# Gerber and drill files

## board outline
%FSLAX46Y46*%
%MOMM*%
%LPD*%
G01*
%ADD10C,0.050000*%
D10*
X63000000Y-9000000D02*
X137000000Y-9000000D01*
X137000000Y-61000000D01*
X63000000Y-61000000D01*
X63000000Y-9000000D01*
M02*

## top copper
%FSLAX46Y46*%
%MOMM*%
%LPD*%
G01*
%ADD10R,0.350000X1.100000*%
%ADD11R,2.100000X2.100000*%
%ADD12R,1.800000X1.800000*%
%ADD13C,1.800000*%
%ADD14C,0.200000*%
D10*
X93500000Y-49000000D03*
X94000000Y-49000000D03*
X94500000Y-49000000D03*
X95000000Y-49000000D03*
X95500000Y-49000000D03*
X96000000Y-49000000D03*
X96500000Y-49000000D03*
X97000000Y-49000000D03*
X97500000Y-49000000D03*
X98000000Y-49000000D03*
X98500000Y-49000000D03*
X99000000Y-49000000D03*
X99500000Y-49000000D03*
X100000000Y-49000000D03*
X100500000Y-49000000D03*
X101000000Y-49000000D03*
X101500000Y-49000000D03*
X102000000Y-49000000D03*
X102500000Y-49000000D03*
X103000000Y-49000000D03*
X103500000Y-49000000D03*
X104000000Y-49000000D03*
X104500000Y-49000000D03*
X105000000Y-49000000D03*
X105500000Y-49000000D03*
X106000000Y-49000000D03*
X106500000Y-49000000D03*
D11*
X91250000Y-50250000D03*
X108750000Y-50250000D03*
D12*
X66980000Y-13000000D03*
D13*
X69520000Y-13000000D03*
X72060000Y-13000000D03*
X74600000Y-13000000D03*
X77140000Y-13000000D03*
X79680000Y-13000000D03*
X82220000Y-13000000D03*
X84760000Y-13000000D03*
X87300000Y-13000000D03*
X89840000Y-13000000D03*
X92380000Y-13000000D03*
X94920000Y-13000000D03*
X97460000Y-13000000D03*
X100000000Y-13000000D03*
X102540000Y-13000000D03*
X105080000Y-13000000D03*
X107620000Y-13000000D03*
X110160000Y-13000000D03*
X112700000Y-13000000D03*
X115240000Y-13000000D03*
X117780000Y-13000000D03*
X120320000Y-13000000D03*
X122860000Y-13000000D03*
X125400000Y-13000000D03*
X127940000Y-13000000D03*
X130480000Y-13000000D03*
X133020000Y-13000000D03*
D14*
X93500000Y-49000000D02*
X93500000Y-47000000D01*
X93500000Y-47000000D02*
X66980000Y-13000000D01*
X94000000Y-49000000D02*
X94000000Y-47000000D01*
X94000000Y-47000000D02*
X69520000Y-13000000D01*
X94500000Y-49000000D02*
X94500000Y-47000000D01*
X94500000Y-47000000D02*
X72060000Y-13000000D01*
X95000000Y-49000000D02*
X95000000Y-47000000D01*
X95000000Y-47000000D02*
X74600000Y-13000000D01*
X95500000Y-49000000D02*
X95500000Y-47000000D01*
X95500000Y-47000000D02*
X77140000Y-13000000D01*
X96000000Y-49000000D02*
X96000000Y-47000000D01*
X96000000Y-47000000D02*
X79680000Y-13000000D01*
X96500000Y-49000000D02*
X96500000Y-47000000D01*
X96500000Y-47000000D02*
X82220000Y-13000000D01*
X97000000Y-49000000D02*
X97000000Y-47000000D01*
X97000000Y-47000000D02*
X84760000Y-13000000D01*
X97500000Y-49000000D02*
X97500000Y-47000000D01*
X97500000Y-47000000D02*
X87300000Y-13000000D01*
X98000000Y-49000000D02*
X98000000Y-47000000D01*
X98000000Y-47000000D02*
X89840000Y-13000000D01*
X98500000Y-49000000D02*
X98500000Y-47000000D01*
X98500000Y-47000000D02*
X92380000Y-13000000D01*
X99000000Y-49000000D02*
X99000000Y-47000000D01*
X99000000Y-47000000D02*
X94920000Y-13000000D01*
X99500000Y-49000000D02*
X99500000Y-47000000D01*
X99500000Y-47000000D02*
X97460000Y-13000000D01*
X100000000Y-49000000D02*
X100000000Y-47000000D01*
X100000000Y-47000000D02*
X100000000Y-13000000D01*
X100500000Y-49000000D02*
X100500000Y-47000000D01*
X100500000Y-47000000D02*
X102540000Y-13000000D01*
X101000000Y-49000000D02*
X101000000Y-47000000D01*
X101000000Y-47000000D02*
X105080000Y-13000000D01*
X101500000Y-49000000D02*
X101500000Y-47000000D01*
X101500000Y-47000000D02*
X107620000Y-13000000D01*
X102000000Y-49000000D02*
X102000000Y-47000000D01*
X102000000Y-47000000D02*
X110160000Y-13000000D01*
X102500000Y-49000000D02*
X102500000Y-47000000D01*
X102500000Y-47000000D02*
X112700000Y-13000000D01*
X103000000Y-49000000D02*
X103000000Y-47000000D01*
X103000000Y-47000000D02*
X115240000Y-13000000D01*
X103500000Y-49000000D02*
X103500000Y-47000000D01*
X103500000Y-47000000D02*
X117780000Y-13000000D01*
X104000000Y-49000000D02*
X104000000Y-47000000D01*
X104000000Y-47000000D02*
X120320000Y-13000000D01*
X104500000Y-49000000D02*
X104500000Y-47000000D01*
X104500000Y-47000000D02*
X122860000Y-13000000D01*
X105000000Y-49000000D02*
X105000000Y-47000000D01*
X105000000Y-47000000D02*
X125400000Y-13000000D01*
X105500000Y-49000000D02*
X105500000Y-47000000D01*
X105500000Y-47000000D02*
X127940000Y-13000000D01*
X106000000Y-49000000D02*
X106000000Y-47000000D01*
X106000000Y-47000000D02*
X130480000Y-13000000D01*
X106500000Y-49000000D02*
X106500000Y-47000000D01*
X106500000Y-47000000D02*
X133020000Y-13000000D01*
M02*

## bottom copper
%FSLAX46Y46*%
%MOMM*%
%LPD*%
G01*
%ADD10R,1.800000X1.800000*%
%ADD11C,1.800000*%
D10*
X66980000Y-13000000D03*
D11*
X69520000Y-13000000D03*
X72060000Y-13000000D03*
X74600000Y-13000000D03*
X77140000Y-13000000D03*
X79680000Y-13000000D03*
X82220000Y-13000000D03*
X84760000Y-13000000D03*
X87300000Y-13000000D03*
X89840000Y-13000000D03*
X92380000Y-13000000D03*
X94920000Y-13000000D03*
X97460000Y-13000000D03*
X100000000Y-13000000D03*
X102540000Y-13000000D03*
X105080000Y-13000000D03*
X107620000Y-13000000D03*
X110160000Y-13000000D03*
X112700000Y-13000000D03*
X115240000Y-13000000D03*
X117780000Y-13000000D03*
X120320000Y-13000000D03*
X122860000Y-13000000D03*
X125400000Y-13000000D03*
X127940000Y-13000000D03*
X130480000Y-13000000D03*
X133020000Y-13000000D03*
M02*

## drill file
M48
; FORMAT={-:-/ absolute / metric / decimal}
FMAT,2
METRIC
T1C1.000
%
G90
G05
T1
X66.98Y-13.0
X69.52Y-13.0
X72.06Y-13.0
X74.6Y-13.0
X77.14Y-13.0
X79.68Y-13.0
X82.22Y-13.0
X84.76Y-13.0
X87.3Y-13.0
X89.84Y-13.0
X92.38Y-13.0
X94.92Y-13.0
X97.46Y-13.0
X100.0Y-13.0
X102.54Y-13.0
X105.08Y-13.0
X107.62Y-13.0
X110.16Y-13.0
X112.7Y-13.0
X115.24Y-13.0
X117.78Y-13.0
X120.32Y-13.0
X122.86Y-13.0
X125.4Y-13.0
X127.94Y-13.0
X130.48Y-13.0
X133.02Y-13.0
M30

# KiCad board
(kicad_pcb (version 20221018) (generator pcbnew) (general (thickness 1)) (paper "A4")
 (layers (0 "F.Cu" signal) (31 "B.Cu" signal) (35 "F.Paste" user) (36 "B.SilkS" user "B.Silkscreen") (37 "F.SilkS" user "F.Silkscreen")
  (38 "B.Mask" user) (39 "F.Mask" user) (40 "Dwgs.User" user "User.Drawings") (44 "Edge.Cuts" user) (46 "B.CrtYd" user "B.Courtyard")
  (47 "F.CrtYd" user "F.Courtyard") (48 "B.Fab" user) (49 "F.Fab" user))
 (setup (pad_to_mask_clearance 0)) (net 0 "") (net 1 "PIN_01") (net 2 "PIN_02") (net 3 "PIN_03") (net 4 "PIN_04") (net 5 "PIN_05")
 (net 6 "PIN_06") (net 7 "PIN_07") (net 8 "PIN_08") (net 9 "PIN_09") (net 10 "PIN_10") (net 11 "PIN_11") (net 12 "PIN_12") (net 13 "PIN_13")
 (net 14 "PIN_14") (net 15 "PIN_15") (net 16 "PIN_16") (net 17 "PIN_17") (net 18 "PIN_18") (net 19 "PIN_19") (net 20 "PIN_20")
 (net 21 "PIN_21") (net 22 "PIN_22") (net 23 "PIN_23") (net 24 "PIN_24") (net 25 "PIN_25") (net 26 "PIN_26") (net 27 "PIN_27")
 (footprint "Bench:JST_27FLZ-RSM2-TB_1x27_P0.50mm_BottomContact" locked (layer "F.Cu") (at 100 49)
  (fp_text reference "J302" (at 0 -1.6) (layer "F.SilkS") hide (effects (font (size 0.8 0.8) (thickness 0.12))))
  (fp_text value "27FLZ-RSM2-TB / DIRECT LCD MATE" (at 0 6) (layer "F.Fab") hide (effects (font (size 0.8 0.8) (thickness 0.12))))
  (pad "1" smd rect locked (at -6.5 0) (size 0.35 1.1) (layers "F.Cu" "F.Paste" "F.Mask") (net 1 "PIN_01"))
  (pad "2" smd rect locked (at -6 0) (size 0.35 1.1) (layers "F.Cu" "F.Paste" "F.Mask") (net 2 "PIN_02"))
  (pad "3" smd rect locked (at -5.5 0) (size 0.35 1.1) (layers "F.Cu" "F.Paste" "F.Mask") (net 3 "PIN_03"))
  (pad "4" smd rect locked (at -5 0) (size 0.35 1.1) (layers "F.Cu" "F.Paste" "F.Mask") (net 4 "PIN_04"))
  (pad "5" smd rect locked (at -4.5 0) (size 0.35 1.1) (layers "F.Cu" "F.Paste" "F.Mask") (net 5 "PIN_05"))
  (pad "6" smd rect locked (at -4 0) (size 0.35 1.1) (layers "F.Cu" "F.Paste" "F.Mask") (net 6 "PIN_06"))
  (pad "7" smd rect locked (at -3.5 0) (size 0.35 1.1) (layers "F.Cu" "F.Paste" "F.Mask") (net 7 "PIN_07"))
  (pad "8" smd rect locked (at -3 0) (size 0.35 1.1) (layers "F.Cu" "F.Paste" "F.Mask") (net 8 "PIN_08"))
  (pad "9" smd rect locked (at -2.5 0) (size 0.35 1.1) (layers "F.Cu" "F.Paste" "F.Mask") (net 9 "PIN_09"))
  (pad "10" smd rect locked (at -2 0) (size 0.35 1.1) (layers "F.Cu" "F.Paste" "F.Mask") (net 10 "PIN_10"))
  (pad "11" smd rect locked (at -1.5 0) (size 0.35 1.1) (layers "F.Cu" "F.Paste" "F.Mask") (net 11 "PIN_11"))
  (pad "12" smd rect locked (at -1 0) (size 0.35 1.1) (layers "F.Cu" "F.Paste" "F.Mask") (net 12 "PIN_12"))
  (pad "13" smd rect locked (at -0.5 0) (size 0.35 1.1) (layers "F.Cu" "F.Paste" "F.Mask") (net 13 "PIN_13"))
  (pad "14" smd rect locked (at 0 0) (size 0.35 1.1) (layers "F.Cu" "F.Paste" "F.Mask") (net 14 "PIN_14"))
  (pad "15" smd rect locked (at 0.5 0) (size 0.35 1.1) (layers "F.Cu" "F.Paste" "F.Mask") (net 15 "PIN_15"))
  (pad "16" smd rect locked (at 1 0) (size 0.35 1.1) (layers "F.Cu" "F.Paste" "F.Mask") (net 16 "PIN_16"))
  (pad "17" smd rect locked (at 1.5 0) (size 0.35 1.1) (layers "F.Cu" "F.Paste" "F.Mask") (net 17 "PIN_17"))
  (pad "18" smd rect locked (at 2 0) (size 0.35 1.1) (layers "F.Cu" "F.Paste" "F.Mask") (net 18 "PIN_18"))
  (pad "19" smd rect locked (at 2.5 0) (size 0.35 1.1) (layers "F.Cu" "F.Paste" "F.Mask") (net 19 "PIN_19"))
  (pad "20" smd rect locked (at 3 0) (size 0.35 1.1) (layers "F.Cu" "F.Paste" "F.Mask") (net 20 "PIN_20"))
  (pad "21" smd rect locked (at 3.5 0) (size 0.35 1.1) (layers "F.Cu" "F.Paste" "F.Mask") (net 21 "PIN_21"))
  (pad "22" smd rect locked (at 4 0) (size 0.35 1.1) (layers "F.Cu" "F.Paste" "F.Mask") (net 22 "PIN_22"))
  (pad "23" smd rect locked (at 4.5 0) (size 0.35 1.1) (layers "F.Cu" "F.Paste" "F.Mask") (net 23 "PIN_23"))
  (pad "24" smd rect locked (at 5 0) (size 0.35 1.1) (layers "F.Cu" "F.Paste" "F.Mask") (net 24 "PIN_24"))
  (pad "25" smd rect locked (at 5.5 0) (size 0.35 1.1) (layers "F.Cu" "F.Paste" "F.Mask") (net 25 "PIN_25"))
  (pad "26" smd rect locked (at 6 0) (size 0.35 1.1) (layers "F.Cu" "F.Paste" "F.Mask") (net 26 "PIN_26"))
  (pad "27" smd rect locked (at 6.5 0) (size 0.35 1.1) (layers "F.Cu" "F.Paste" "F.Mask") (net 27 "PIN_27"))
  (pad "MP" smd rect locked (at -8.75 1.25) (size 2.1 2.1) (layers "F.Cu" "F.Paste" "F.Mask"))
  (pad "MP" smd rect locked (at 8.75 1.25) (size 2.1 2.1) (layers "F.Cu" "F.Paste" "F.Mask")))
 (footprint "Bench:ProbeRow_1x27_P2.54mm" (at 100 13) (layer "F.Cu")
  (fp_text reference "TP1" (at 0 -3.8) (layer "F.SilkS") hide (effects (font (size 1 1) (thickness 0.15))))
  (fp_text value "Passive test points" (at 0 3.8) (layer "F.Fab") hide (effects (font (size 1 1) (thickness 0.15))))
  (pad "1" thru_hole rect (at -33.02 0) (size 1.8 1.8) (drill 1) (layers "*.Cu" "*.Mask") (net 1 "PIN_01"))
  (pad "2" thru_hole circle (at -30.48 0) (size 1.8 1.8) (drill 1) (layers "*.Cu" "*.Mask") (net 2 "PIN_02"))
  (pad "3" thru_hole circle (at -27.94 0) (size 1.8 1.8) (drill 1) (layers "*.Cu" "*.Mask") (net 3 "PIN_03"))
  (pad "4" thru_hole circle (at -25.40 0) (size 1.8 1.8) (drill 1) (layers "*.Cu" "*.Mask") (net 4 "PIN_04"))
  (pad "5" thru_hole circle (at -22.86 0) (size 1.8 1.8) (drill 1) (layers "*.Cu" "*.Mask") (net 5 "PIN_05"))
  (pad "6" thru_hole circle (at -20.32 0) (size 1.8 1.8) (drill 1) (layers "*.Cu" "*.Mask") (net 6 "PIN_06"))
  (pad "7" thru_hole circle (at -17.78 0) (size 1.8 1.8) (drill 1) (layers "*.Cu" "*.Mask") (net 7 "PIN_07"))
  (pad "8" thru_hole circle (at -15.24 0) (size 1.8 1.8) (drill 1) (layers "*.Cu" "*.Mask") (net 8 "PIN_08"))
  (pad "9" thru_hole circle (at -12.70 0) (size 1.8 1.8) (drill 1) (layers "*.Cu" "*.Mask") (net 9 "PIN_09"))
  (pad "10" thru_hole circle (at -10.16 0) (size 1.8 1.8) (drill 1) (layers "*.Cu" "*.Mask") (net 10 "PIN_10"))
  (pad "11" thru_hole circle (at -7.62 0) (size 1.8 1.8) (drill 1) (layers "*.Cu" "*.Mask") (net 11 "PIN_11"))
  (pad "12" thru_hole circle (at -5.08 0) (size 1.8 1.8) (drill 1) (layers "*.Cu" "*.Mask") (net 12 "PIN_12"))
  (pad "13" thru_hole circle (at -2.54 0) (size 1.8 1.8) (drill 1) (layers "*.Cu" "*.Mask") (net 13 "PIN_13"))
  (pad "14" thru_hole circle (at 0.00 0) (size 1.8 1.8) (drill 1) (layers "*.Cu" "*.Mask") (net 14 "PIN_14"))
  (pad "15" thru_hole circle (at 2.54 0) (size 1.8 1.8) (drill 1) (layers "*.Cu" "*.Mask") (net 15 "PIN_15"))
  (pad "16" thru_hole circle (at 5.08 0) (size 1.8 1.8) (drill 1) (layers "*.Cu" "*.Mask") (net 16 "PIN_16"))
  (pad "17" thru_hole circle (at 7.62 0) (size 1.8 1.8) (drill 1) (layers "*.Cu" "*.Mask") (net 17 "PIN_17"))
  (pad "18" thru_hole circle (at 10.16 0) (size 1.8 1.8) (drill 1) (layers "*.Cu" "*.Mask") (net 18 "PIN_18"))
  (pad "19" thru_hole circle (at 12.70 0) (size 1.8 1.8) (drill 1) (layers "*.Cu" "*.Mask") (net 19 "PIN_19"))
  (pad "20" thru_hole circle (at 15.24 0) (size 1.8 1.8) (drill 1) (layers "*.Cu" "*.Mask") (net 20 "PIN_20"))
  (pad "21" thru_hole circle (at 17.78 0) (size 1.8 1.8) (drill 1) (layers "*.Cu" "*.Mask") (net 21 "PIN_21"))
  (pad "22" thru_hole circle (at 20.32 0) (size 1.8 1.8) (drill 1) (layers "*.Cu" "*.Mask") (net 22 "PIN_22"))
  (pad "23" thru_hole circle (at 22.86 0) (size 1.8 1.8) (drill 1) (layers "*.Cu" "*.Mask") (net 23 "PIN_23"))
  (pad "24" thru_hole circle (at 25.40 0) (size 1.8 1.8) (drill 1) (layers "*.Cu" "*.Mask") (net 24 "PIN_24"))
  (pad "25" thru_hole circle (at 27.94 0) (size 1.8 1.8) (drill 1) (layers "*.Cu" "*.Mask") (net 25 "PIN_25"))
  (pad "26" thru_hole circle (at 30.48 0) (size 1.8 1.8) (drill 1) (layers "*.Cu" "*.Mask") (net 26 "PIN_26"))
  (pad "27" thru_hole circle (at 33.02 0) (size 1.8 1.8) (drill 1) (layers "*.Cu" "*.Mask") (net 27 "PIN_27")))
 (gr_rect (start 63 9) (end 137 61) (stroke (width 0.05) (type default)) (fill none) (layer "Edge.Cuts"))
 (segment (start 93.50000 49.00000) (end 93.50000 47.00000) (width 0.20) (layer "F.Cu") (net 1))
 (segment (start 93.50000 47.00000) (end 66.98000 13.00000) (width 0.20) (layer "F.Cu") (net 1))
 (segment (start 94.00000 49.00000) (end 94.00000 47.00000) (width 0.20) (layer "F.Cu") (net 2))
 (segment (start 94.00000 47.00000) (end 69.52000 13.00000) (width 0.20) (layer "F.Cu") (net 2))
 (segment (start 94.50000 49.00000) (end 94.50000 47.00000) (width 0.20) (layer "F.Cu") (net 3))
 (segment (start 94.50000 47.00000) (end 72.06000 13.00000) (width 0.20) (layer "F.Cu") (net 3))
 (segment (start 95.00000 49.00000) (end 95.00000 47.00000) (width 0.20) (layer "F.Cu") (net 4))
 (segment (start 95.00000 47.00000) (end 74.60000 13.00000) (width 0.20) (layer "F.Cu") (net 4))
 (segment (start 95.50000 49.00000) (end 95.50000 47.00000) (width 0.20) (layer "F.Cu") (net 5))
 (segment (start 95.50000 47.00000) (end 77.14000 13.00000) (width 0.20) (layer "F.Cu") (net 5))
 (segment (start 96.00000 49.00000) (end 96.00000 47.00000) (width 0.20) (layer "F.Cu") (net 6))
 (segment (start 96.00000 47.00000) (end 79.68000 13.00000) (width 0.20) (layer "F.Cu") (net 6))
 (segment (start 96.50000 49.00000) (end 96.50000 47.00000) (width 0.20) (layer "F.Cu") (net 7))
 (segment (start 96.50000 47.00000) (end 82.22000 13.00000) (width 0.20) (layer "F.Cu") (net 7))
 (segment (start 97.00000 49.00000) (end 97.00000 47.00000) (width 0.20) (layer "F.Cu") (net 8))
 (segment (start 97.00000 47.00000) (end 84.76000 13.00000) (width 0.20) (layer "F.Cu") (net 8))
 (segment (start 97.50000 49.00000) (end 97.50000 47.00000) (width 0.20) (layer "F.Cu") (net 9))
 (segment (start 97.50000 47.00000) (end 87.30000 13.00000) (width 0.20) (layer "F.Cu") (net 9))
 (segment (start 98.00000 49.00000) (end 98.00000 47.00000) (width 0.20) (layer "F.Cu") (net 10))
 (segment (start 98.00000 47.00000) (end 89.84000 13.00000) (width 0.20) (layer "F.Cu") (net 10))
 (segment (start 98.50000 49.00000) (end 98.50000 47.00000) (width 0.20) (layer "F.Cu") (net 11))
 (segment (start 98.50000 47.00000) (end 92.38000 13.00000) (width 0.20) (layer "F.Cu") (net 11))
 (segment (start 99.00000 49.00000) (end 99.00000 47.00000) (width 0.20) (layer "F.Cu") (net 12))
 (segment (start 99.00000 47.00000) (end 94.92000 13.00000) (width 0.20) (layer "F.Cu") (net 12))
 (segment (start 99.50000 49.00000) (end 99.50000 47.00000) (width 0.20) (layer "F.Cu") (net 13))
 (segment (start 99.50000 47.00000) (end 97.46000 13.00000) (width 0.20) (layer "F.Cu") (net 13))
 (segment (start 100.00000 49.00000) (end 100.00000 47.00000) (width 0.20) (layer "F.Cu") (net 14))
 (segment (start 100.00000 47.00000) (end 100.00000 13.00000) (width 0.20) (layer "F.Cu") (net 14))
 (segment (start 100.50000 49.00000) (end 100.50000 47.00000) (width 0.20) (layer "F.Cu") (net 15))
 (segment (start 100.50000 47.00000) (end 102.54000 13.00000) (width 0.20) (layer "F.Cu") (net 15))
 (segment (start 101.00000 49.00000) (end 101.00000 47.00000) (width 0.20) (layer "F.Cu") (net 16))
 (segment (start 101.00000 47.00000) (end 105.08000 13.00000) (width 0.20) (layer "F.Cu") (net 16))
 (segment (start 101.50000 49.00000) (end 101.50000 47.00000) (width 0.20) (layer "F.Cu") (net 17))
 (segment (start 101.50000 47.00000) (end 107.62000 13.00000) (width 0.20) (layer "F.Cu") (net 17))
 (segment (start 102.00000 49.00000) (end 102.00000 47.00000) (width 0.20) (layer "F.Cu") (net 18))
 (segment (start 102.00000 47.00000) (end 110.16000 13.00000) (width 0.20) (layer "F.Cu") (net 18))
 (segment (start 102.50000 49.00000) (end 102.50000 47.00000) (width 0.20) (layer "F.Cu") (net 19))
 (segment (start 102.50000 47.00000) (end 112.70000 13.00000) (width 0.20) (layer "F.Cu") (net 19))
 (segment (start 103.00000 49.00000) (end 103.00000 47.00000) (width 0.20) (layer "F.Cu") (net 20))
 (segment (start 103.00000 47.00000) (end 115.24000 13.00000) (width 0.20) (layer "F.Cu") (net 20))
 (segment (start 103.50000 49.00000) (end 103.50000 47.00000) (width 0.20) (layer "F.Cu") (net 21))
 (segment (start 103.50000 47.00000) (end 117.78000 13.00000) (width 0.20) (layer "F.Cu") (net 21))
 (segment (start 104.00000 49.00000) (end 104.00000 47.00000) (width 0.20) (layer "F.Cu") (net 22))
 (segment (start 104.00000 47.00000) (end 120.32000 13.00000) (width 0.20) (layer "F.Cu") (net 22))
 (segment (start 104.50000 49.00000) (end 104.50000 47.00000) (width 0.20) (layer "F.Cu") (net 23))
 (segment (start 104.50000 47.00000) (end 122.86000 13.00000) (width 0.20) (layer "F.Cu") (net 23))
 (segment (start 105.00000 49.00000) (end 105.00000 47.00000) (width 0.20) (layer "F.Cu") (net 24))
 (segment (start 105.00000 47.00000) (end 125.40000 13.00000) (width 0.20) (layer "F.Cu") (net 24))
 (segment (start 105.50000 49.00000) (end 105.50000 47.00000) (width 0.20) (layer "F.Cu") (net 25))
 (segment (start 105.50000 47.00000) (end 127.94000 13.00000) (width 0.20) (layer "F.Cu") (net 25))
 (segment (start 106.00000 49.00000) (end 106.00000 47.00000) (width 0.20) (layer "F.Cu") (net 26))
 (segment (start 106.00000 47.00000) (end 130.48000 13.00000) (width 0.20) (layer "F.Cu") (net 26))
 (segment (start 106.50000 49.00000) (end 106.50000 47.00000) (width 0.20) (layer "F.Cu") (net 27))
 (segment (start 106.50000 47.00000) (end 133.02000 13.00000) (width 0.20) (layer "F.Cu") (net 27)))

